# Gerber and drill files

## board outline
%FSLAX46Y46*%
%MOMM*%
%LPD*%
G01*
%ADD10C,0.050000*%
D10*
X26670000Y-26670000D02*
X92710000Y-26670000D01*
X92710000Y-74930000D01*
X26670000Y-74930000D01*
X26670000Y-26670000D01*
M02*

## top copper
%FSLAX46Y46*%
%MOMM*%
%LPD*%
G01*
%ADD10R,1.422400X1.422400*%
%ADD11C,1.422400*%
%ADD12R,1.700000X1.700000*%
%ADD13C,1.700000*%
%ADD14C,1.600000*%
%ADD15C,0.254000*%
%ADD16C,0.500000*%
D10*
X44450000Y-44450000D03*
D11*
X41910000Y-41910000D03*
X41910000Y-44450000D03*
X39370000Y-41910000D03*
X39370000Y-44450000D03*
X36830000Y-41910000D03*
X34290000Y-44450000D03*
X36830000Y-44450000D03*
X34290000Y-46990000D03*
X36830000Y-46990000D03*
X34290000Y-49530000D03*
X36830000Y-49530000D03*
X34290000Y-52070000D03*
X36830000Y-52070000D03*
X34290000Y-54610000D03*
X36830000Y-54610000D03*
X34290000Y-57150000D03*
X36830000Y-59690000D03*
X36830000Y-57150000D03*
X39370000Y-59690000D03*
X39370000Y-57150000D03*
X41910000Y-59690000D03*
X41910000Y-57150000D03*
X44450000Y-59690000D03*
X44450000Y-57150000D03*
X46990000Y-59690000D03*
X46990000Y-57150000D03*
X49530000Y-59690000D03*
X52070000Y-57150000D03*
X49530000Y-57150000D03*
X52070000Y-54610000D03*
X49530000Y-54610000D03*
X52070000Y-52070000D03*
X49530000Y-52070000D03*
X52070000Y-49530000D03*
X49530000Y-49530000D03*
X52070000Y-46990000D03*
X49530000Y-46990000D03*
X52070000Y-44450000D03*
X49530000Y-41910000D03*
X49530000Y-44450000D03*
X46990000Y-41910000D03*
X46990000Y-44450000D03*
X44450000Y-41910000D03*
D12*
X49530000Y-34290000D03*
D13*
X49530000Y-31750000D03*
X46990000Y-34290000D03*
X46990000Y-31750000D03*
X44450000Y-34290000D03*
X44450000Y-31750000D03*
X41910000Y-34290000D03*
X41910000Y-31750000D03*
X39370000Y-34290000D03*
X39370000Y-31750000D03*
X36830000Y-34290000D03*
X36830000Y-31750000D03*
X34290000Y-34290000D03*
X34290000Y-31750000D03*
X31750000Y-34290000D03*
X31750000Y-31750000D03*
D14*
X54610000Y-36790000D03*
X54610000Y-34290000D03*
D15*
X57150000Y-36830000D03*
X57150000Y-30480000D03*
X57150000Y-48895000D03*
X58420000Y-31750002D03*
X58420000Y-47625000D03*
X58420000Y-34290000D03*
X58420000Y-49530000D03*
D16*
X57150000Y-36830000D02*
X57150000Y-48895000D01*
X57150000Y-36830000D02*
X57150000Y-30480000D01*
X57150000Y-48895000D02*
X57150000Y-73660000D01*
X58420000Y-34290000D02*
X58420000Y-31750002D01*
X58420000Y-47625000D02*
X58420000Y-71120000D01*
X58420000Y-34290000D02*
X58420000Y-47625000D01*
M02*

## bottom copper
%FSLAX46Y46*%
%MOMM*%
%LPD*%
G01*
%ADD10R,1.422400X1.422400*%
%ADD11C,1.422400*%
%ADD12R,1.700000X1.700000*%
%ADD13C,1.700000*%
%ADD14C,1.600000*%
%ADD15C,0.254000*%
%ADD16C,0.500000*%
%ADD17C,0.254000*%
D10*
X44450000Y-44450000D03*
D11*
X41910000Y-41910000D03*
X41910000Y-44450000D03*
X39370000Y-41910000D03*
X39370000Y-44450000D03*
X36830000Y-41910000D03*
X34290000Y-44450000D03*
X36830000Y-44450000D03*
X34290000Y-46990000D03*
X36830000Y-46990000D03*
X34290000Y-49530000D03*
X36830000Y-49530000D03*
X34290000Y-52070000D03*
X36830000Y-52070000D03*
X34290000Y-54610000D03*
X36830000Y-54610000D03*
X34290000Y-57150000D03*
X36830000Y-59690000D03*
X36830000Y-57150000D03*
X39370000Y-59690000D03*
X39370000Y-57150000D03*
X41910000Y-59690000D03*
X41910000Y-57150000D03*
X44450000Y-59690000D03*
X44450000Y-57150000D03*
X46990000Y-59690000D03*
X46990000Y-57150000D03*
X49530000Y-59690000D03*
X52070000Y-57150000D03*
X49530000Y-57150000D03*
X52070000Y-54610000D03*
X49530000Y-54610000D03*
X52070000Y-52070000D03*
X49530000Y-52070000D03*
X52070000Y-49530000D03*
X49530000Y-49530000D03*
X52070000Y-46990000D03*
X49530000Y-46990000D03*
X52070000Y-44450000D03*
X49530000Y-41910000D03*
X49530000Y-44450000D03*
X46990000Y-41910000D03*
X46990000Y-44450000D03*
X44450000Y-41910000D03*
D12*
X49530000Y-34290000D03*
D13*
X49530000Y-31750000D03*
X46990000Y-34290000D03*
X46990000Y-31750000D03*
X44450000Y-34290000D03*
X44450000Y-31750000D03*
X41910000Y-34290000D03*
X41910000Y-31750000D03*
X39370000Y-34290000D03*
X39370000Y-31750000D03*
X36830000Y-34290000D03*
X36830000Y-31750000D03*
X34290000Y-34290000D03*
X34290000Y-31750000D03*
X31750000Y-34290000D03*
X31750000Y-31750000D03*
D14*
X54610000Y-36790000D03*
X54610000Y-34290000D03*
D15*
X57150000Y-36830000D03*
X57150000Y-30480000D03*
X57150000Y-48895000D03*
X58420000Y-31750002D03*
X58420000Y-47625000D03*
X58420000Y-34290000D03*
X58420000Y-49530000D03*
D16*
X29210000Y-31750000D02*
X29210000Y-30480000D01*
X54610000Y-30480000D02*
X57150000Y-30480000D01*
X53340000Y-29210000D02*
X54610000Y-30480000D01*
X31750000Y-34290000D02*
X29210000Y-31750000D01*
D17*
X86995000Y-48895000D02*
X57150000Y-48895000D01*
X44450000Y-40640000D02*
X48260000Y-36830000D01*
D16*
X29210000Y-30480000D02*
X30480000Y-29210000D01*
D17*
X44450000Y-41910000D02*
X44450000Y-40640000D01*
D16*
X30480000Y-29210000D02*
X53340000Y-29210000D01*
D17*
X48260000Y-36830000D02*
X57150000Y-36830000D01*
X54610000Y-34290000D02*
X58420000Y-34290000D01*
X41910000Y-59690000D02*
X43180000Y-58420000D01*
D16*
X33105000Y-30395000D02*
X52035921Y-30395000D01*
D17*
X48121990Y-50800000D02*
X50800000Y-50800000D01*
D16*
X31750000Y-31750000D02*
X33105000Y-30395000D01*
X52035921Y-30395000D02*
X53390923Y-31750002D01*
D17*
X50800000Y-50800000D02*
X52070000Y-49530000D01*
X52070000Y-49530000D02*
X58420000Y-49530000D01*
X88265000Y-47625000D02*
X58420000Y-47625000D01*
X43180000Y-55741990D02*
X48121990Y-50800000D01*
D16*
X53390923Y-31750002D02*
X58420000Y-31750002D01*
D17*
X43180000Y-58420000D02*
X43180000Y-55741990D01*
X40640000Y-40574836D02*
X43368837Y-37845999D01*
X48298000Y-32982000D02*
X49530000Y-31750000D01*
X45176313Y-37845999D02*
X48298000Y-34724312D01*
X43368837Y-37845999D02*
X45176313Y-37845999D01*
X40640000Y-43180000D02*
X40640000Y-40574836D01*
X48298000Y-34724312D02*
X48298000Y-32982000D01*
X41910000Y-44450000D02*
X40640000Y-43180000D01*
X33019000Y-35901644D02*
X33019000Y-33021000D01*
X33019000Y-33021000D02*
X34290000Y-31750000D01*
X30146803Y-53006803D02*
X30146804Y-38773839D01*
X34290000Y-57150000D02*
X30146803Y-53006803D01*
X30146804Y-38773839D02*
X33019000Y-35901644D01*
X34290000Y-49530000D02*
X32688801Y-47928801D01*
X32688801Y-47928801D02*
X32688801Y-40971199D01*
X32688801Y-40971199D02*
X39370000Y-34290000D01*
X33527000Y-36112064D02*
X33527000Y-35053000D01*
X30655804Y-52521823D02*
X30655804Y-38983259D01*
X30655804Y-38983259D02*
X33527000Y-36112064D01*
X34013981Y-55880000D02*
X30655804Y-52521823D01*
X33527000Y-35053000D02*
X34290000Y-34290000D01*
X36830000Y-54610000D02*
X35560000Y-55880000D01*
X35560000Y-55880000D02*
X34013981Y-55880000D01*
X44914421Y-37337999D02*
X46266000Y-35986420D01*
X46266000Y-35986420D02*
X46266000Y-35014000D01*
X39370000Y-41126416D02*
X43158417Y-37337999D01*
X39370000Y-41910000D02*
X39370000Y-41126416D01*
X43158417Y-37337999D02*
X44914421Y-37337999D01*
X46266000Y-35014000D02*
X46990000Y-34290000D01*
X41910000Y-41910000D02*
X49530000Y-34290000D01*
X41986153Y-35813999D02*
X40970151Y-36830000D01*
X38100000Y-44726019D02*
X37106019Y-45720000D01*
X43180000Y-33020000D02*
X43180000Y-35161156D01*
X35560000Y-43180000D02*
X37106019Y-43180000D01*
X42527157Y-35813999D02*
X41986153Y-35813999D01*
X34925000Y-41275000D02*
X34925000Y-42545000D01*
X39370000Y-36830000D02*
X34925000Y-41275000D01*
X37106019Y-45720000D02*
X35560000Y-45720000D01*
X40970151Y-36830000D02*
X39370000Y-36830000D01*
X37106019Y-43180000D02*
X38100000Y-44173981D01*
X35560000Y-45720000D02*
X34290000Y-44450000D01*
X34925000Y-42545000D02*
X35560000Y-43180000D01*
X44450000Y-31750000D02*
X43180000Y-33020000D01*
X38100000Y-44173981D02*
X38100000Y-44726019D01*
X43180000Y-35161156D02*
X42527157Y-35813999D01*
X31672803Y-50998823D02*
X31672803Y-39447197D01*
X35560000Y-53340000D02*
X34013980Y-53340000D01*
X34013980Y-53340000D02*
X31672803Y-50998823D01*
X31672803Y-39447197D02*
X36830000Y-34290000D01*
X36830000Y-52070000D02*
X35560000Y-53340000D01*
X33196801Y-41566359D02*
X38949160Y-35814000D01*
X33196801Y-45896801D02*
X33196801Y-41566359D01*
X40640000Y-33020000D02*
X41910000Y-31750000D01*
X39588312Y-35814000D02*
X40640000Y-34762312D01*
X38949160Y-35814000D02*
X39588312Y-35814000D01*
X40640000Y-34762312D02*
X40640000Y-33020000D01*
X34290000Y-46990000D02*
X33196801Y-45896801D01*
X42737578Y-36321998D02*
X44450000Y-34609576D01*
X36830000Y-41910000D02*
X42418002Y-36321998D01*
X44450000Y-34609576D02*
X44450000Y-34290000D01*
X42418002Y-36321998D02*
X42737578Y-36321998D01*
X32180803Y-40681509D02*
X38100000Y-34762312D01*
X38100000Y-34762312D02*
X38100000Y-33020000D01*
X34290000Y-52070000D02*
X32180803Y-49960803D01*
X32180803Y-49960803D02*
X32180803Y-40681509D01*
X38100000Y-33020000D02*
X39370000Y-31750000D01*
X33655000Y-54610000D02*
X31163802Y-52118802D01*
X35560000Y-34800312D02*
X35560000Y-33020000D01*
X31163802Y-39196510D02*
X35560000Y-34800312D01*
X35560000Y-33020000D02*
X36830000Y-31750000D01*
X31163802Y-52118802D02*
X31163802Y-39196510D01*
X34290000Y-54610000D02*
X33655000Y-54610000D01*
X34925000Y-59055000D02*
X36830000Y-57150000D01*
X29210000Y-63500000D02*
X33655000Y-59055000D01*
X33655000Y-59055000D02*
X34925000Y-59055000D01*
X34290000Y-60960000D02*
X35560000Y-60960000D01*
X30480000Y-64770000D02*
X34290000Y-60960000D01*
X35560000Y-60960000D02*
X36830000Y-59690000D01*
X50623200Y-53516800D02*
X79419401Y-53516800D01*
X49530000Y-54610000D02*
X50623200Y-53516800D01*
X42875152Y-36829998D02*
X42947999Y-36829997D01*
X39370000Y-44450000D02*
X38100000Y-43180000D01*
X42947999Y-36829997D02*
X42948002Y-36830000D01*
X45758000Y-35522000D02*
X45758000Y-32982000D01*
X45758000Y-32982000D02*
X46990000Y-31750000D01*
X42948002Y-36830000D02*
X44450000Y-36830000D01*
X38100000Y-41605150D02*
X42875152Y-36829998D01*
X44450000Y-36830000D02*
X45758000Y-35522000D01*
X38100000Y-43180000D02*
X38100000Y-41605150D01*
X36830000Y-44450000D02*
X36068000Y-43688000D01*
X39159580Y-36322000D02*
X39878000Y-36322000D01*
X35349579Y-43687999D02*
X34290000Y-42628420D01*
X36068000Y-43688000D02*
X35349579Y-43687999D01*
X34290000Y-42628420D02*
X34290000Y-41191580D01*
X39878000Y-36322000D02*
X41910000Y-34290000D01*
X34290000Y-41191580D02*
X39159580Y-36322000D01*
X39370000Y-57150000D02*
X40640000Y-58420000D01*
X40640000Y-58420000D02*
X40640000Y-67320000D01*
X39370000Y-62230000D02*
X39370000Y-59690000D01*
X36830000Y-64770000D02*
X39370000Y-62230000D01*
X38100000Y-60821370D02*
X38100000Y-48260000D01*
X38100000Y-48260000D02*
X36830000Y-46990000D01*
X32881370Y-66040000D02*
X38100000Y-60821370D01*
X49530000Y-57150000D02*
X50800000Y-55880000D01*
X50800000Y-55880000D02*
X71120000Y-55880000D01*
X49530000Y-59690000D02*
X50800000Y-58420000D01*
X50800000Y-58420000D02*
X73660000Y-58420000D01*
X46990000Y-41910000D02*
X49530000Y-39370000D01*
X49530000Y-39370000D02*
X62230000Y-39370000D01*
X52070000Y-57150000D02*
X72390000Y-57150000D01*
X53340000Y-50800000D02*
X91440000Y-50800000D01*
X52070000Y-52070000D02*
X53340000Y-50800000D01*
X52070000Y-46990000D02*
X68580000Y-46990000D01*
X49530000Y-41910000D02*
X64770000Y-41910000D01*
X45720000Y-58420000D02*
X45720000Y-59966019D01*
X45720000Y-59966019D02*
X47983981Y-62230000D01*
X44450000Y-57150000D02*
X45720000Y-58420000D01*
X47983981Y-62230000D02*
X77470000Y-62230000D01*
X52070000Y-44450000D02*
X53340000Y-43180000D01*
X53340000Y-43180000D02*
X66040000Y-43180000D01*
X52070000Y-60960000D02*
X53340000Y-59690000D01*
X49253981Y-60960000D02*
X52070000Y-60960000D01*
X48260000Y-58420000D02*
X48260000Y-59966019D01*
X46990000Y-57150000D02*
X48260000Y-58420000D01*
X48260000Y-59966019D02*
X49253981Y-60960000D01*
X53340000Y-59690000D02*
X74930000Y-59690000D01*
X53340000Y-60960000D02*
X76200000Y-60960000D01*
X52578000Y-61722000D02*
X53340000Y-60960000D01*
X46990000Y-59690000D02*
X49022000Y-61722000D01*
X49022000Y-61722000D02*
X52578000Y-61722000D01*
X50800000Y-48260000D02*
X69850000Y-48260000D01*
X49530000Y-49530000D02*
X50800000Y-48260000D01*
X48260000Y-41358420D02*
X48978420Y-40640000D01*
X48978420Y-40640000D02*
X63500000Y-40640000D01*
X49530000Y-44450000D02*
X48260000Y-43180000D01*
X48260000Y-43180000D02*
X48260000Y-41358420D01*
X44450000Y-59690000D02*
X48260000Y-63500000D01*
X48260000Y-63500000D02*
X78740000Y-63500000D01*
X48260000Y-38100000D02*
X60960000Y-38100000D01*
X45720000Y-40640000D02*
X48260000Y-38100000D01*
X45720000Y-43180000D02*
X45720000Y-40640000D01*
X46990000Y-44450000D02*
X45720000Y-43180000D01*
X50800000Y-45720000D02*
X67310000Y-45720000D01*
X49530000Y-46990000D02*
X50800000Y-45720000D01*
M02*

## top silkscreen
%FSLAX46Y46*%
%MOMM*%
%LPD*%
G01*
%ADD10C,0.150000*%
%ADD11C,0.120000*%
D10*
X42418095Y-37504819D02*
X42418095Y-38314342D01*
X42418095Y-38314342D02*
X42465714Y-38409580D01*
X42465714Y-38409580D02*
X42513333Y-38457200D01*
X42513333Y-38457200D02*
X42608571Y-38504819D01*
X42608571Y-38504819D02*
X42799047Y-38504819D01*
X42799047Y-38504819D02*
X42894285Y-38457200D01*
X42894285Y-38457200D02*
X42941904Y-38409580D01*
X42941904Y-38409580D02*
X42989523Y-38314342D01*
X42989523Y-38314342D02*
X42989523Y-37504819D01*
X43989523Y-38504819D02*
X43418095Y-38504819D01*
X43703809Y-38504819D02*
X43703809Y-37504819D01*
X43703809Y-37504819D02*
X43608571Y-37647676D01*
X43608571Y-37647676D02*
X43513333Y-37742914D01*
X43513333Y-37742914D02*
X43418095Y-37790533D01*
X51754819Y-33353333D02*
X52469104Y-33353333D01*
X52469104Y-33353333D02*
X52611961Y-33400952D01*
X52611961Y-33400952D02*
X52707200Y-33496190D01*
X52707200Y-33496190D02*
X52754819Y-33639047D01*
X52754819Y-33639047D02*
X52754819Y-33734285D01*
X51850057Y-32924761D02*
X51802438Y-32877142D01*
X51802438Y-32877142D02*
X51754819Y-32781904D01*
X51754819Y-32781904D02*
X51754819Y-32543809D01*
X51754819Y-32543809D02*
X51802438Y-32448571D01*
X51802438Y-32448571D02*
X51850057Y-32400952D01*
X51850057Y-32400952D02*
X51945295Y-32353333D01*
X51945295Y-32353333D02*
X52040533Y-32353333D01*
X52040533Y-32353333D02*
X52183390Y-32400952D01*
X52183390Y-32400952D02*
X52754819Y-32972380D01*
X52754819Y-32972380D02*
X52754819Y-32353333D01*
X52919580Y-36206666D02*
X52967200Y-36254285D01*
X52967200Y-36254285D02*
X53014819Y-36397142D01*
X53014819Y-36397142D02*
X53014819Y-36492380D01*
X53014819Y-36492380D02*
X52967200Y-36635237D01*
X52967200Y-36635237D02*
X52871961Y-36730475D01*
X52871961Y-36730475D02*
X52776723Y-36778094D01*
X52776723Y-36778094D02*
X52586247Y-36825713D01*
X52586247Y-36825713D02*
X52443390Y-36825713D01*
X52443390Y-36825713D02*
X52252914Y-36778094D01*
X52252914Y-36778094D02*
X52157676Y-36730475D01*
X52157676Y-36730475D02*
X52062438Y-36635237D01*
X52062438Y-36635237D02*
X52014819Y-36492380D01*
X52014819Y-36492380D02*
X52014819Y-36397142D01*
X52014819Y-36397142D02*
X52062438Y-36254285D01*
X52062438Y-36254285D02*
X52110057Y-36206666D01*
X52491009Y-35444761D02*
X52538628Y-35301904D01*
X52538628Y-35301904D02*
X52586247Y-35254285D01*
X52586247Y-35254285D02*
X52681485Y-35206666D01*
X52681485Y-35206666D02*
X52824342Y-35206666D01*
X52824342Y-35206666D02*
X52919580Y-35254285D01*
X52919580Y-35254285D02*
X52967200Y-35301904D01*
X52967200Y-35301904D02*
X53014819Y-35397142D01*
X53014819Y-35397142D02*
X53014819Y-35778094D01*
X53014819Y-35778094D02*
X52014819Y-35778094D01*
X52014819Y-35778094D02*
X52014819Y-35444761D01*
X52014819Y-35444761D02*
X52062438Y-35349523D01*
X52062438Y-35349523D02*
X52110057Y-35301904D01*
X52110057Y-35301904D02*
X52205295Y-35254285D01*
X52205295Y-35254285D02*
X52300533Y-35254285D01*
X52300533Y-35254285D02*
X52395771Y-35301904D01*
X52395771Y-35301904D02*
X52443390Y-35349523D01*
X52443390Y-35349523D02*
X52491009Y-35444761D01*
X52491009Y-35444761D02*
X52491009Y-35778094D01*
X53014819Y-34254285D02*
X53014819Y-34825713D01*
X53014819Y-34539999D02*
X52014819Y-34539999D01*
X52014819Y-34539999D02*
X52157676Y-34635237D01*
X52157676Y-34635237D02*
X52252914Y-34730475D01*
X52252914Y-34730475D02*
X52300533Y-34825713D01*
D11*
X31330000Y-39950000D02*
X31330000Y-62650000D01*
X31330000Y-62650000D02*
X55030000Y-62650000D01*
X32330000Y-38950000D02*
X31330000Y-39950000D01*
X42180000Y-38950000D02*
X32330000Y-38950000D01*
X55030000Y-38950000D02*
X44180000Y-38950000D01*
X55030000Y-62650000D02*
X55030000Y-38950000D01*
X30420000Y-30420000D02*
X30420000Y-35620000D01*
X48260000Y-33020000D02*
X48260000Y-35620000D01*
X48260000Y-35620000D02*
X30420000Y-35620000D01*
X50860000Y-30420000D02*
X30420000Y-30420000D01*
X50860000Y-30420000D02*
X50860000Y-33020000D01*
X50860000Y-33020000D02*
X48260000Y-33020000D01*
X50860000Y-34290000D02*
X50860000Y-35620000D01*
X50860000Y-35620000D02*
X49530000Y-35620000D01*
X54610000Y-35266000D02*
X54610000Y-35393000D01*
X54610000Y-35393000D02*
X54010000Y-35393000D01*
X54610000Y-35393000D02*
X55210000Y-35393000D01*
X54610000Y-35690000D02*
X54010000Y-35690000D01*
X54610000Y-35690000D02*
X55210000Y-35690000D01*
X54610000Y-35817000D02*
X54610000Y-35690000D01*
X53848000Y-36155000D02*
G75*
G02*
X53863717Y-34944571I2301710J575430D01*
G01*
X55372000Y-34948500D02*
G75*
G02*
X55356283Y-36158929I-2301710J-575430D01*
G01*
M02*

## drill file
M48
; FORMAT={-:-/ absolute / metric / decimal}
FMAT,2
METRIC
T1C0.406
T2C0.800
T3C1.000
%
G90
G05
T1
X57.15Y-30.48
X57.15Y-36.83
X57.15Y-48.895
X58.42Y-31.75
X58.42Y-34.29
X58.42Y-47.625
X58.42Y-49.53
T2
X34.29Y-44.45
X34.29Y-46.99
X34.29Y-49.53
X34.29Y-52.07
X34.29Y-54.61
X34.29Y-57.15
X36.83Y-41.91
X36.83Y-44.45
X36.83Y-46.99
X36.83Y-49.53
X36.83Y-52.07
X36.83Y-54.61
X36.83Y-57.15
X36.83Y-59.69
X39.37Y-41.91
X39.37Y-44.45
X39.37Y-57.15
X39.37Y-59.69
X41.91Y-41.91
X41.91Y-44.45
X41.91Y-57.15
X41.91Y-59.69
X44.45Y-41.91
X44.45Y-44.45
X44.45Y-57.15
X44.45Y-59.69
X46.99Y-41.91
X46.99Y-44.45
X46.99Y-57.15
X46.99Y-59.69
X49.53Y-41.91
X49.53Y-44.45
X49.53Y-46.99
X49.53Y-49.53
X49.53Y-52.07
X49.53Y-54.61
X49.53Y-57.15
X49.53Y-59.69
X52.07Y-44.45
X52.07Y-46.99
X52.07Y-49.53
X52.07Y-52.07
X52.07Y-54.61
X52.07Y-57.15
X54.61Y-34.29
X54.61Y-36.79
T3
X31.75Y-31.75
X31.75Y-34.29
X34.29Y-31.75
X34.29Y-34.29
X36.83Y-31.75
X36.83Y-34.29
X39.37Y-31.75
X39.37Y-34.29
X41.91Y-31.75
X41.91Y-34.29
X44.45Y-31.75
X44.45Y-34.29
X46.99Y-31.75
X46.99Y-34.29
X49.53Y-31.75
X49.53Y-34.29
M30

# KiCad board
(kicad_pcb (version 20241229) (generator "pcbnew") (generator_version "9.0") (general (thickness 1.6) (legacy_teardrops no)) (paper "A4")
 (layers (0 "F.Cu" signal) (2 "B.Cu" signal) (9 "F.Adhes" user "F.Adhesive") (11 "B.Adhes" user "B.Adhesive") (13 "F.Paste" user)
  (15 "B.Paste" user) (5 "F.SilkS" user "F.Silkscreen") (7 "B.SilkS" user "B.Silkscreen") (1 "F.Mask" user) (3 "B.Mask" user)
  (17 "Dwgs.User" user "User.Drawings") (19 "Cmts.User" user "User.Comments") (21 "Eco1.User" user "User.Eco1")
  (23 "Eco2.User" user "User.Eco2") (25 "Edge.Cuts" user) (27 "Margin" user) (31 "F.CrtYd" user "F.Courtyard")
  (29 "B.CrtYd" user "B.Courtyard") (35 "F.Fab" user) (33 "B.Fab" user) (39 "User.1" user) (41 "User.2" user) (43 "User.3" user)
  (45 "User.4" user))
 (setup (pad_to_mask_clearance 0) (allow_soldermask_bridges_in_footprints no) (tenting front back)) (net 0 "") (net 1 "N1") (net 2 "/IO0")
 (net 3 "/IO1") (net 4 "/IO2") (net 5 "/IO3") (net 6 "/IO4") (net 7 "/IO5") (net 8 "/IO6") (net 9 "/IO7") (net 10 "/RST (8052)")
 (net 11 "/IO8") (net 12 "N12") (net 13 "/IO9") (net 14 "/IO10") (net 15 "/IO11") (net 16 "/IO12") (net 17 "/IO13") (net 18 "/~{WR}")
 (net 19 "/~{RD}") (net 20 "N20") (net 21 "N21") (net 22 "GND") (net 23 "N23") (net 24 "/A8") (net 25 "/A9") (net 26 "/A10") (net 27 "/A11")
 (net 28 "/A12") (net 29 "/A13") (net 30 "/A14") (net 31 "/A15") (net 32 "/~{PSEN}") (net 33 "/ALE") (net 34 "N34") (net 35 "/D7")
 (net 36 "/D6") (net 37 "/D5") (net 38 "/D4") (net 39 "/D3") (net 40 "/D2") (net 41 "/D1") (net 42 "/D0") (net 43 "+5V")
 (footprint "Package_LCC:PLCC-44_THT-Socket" (layer "F.Cu") (at 44.45 44.45)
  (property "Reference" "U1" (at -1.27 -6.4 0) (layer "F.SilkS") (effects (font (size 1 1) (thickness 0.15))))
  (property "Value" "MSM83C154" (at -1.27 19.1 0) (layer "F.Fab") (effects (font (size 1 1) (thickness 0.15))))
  (fp_line (start -13.12 -4.5) (end -13.12 18.2) (stroke (width 0.12) (type solid)) (layer "F.SilkS"))
  (fp_line (start -13.12 18.2) (end 10.58 18.2) (stroke (width 0.12) (type solid)) (layer "F.SilkS"))
  (fp_line (start -12.12 -5.5) (end -13.12 -4.5) (stroke (width 0.12) (type solid)) (layer "F.SilkS"))
  (fp_line (start -2.27 -5.5) (end -12.12 -5.5) (stroke (width 0.12) (type solid)) (layer "F.SilkS"))
  (fp_line (start 10.58 -5.5) (end -0.27 -5.5) (stroke (width 0.12) (type solid)) (layer "F.SilkS"))
  (fp_line (start 10.58 18.2) (end 10.58 -5.5) (stroke (width 0.12) (type solid)) (layer "F.SilkS"))
  (pad "1" thru_hole rect (at 0 0) (size 1.4224 1.4224) (drill 0.8) (layers "*.Cu" "*.Mask") (remove_unused_layers no) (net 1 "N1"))
  (pad "2" thru_hole circle (at -2.54 -2.54) (size 1.4224 1.4224) (drill 0.8) (layers "*.Cu" "*.Mask") (remove_unused_layers no)
   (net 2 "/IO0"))
  (pad "3" thru_hole circle (at -2.54 0) (size 1.4224 1.4224) (drill 0.8) (layers "*.Cu" "*.Mask") (remove_unused_layers no) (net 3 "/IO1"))
  (pad "4" thru_hole circle (at -5.08 -2.54) (size 1.4224 1.4224) (drill 0.8) (layers "*.Cu" "*.Mask") (remove_unused_layers no)
   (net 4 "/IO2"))
  (pad "5" thru_hole circle (at -5.08 0) (size 1.4224 1.4224) (drill 0.8) (layers "*.Cu" "*.Mask") (remove_unused_layers no) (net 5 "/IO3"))
  (pad "6" thru_hole circle (at -7.62 -2.54) (size 1.4224 1.4224) (drill 0.8) (layers "*.Cu" "*.Mask") (remove_unused_layers no)
   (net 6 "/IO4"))
  (pad "7" thru_hole circle (at -10.16 0) (size 1.4224 1.4224) (drill 0.8) (layers "*.Cu" "*.Mask") (remove_unused_layers no) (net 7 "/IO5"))
  (pad "8" thru_hole circle (at -7.62 0) (size 1.4224 1.4224) (drill 0.8) (layers "*.Cu" "*.Mask") (remove_unused_layers no) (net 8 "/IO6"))
  (pad "9" thru_hole circle (at -10.16 2.54) (size 1.4224 1.4224) (drill 0.8) (layers "*.Cu" "*.Mask") (remove_unused_layers no)
   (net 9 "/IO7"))
  (pad "10" thru_hole circle (at -7.62 2.54) (size 1.4224 1.4224) (drill 0.8) (layers "*.Cu" "*.Mask") (remove_unused_layers no)
   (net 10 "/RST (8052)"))
  (pad "11" thru_hole circle (at -10.16 5.08) (size 1.4224 1.4224) (drill 0.8) (layers "*.Cu" "*.Mask") (remove_unused_layers no)
   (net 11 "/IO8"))
  (pad "12" thru_hole circle (at -7.62 5.08) (size 1.4224 1.4224) (drill 0.8) (layers "*.Cu" "*.Mask") (remove_unused_layers no)
   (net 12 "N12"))
  (pad "13" thru_hole circle (at -10.16 7.62) (size 1.4224 1.4224) (drill 0.8) (layers "*.Cu" "*.Mask") (remove_unused_layers no)
   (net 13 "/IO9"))
  (pad "14" thru_hole circle (at -7.62 7.62) (size 1.4224 1.4224) (drill 0.8) (layers "*.Cu" "*.Mask") (remove_unused_layers no)
   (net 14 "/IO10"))
  (pad "15" thru_hole circle (at -10.16 10.16) (size 1.4224 1.4224) (drill 0.8) (layers "*.Cu" "*.Mask") (remove_unused_layers no)
   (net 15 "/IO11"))
  (pad "16" thru_hole circle (at -7.62 10.16) (size 1.4224 1.4224) (drill 0.8) (layers "*.Cu" "*.Mask") (remove_unused_layers no)
   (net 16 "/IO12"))
  (pad "17" thru_hole circle (at -10.16 12.7) (size 1.4224 1.4224) (drill 0.8) (layers "*.Cu" "*.Mask") (remove_unused_layers no)
   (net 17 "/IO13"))
  (pad "18" thru_hole circle (at -7.62 15.24) (size 1.4224 1.4224) (drill 0.8) (layers "*.Cu" "*.Mask") (remove_unused_layers no)
   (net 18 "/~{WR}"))
  (pad "19" thru_hole circle (at -7.62 12.7) (size 1.4224 1.4224) (drill 0.8) (layers "*.Cu" "*.Mask") (remove_unused_layers no)
   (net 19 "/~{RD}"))
  (pad "20" thru_hole circle (at -5.08 15.24) (size 1.4224 1.4224) (drill 0.8) (layers "*.Cu" "*.Mask") (remove_unused_layers no)
   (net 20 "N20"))
  (pad "21" thru_hole circle (at -5.08 12.7) (size 1.4224 1.4224) (drill 0.8) (layers "*.Cu" "*.Mask") (remove_unused_layers no)
   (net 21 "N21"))
  (pad "22" thru_hole circle (at -2.54 15.24) (size 1.4224 1.4224) (drill 0.8) (layers "*.Cu" "*.Mask") (remove_unused_layers no)
   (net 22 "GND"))
  (pad "23" thru_hole circle (at -2.54 12.7) (size 1.4224 1.4224) (drill 0.8) (layers "*.Cu" "*.Mask") (remove_unused_layers no)
   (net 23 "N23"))
  (pad "24" thru_hole circle (at 0 15.24) (size 1.4224 1.4224) (drill 0.8) (layers "*.Cu" "*.Mask") (remove_unused_layers no) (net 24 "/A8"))
  (pad "25" thru_hole circle (at 0 12.7) (size 1.4224 1.4224) (drill 0.8) (layers "*.Cu" "*.Mask") (remove_unused_layers no) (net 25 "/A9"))
  (pad "26" thru_hole circle (at 2.54 15.24) (size 1.4224 1.4224) (drill 0.8) (layers "*.Cu" "*.Mask") (remove_unused_layers no)
   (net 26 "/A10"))
  (pad "27" thru_hole circle (at 2.54 12.7) (size 1.4224 1.4224) (drill 0.8) (layers "*.Cu" "*.Mask") (remove_unused_layers no)
   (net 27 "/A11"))
  (pad "28" thru_hole circle (at 5.08 15.24) (size 1.4224 1.4224) (drill 0.8) (layers "*.Cu" "*.Mask") (remove_unused_layers no)
   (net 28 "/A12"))
  (pad "29" thru_hole circle (at 7.62 12.7) (size 1.4224 1.4224) (drill 0.8) (layers "*.Cu" "*.Mask") (remove_unused_layers no)
   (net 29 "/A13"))
  (pad "30" thru_hole circle (at 5.08 12.7) (size 1.4224 1.4224) (drill 0.8) (layers "*.Cu" "*.Mask") (remove_unused_layers no)
   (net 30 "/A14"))
  (pad "31" thru_hole circle (at 7.62 10.16) (size 1.4224 1.4224) (drill 0.8) (layers "*.Cu" "*.Mask") (remove_unused_layers no)
   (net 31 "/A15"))
  (pad "32" thru_hole circle (at 5.08 10.16) (size 1.4224 1.4224) (drill 0.8) (layers "*.Cu" "*.Mask") (remove_unused_layers no)
   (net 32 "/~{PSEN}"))
  (pad "33" thru_hole circle (at 7.62 7.62) (size 1.4224 1.4224) (drill 0.8) (layers "*.Cu" "*.Mask") (remove_unused_layers no)
   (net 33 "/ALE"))
  (pad "34" thru_hole circle (at 5.08 7.62) (size 1.4224 1.4224) (drill 0.8) (layers "*.Cu" "*.Mask") (remove_unused_layers no)
   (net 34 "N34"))
  (pad "35" thru_hole circle (at 7.62 5.08) (size 1.4224 1.4224) (drill 0.8) (layers "*.Cu" "*.Mask") (remove_unused_layers no)
   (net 22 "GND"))
  (pad "36" thru_hole circle (at 5.08 5.08) (size 1.4224 1.4224) (drill 0.8) (layers "*.Cu" "*.Mask") (remove_unused_layers no)
   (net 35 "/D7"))
  (pad "37" thru_hole circle (at 7.62 2.54) (size 1.4224 1.4224) (drill 0.8) (layers "*.Cu" "*.Mask") (remove_unused_layers no)
   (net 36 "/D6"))
  (pad "38" thru_hole circle (at 5.08 2.54) (size 1.4224 1.4224) (drill 0.8) (layers "*.Cu" "*.Mask") (remove_unused_layers no)
   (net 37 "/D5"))
  (pad "39" thru_hole circle (at 7.62 0) (size 1.4224 1.4224) (drill 0.8) (layers "*.Cu" "*.Mask") (remove_unused_layers no) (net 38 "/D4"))
  (pad "40" thru_hole circle (at 5.08 -2.54) (size 1.4224 1.4224) (drill 0.8) (layers "*.Cu" "*.Mask") (remove_unused_layers no)
   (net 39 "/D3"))
  (pad "41" thru_hole circle (at 5.08 0) (size 1.4224 1.4224) (drill 0.8) (layers "*.Cu" "*.Mask") (remove_unused_layers no) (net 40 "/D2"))
  (pad "42" thru_hole circle (at 2.54 -2.54) (size 1.4224 1.4224) (drill 0.8) (layers "*.Cu" "*.Mask") (remove_unused_layers no)
   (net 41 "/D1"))
  (pad "43" thru_hole circle (at 2.54 0) (size 1.4224 1.4224) (drill 0.8) (layers "*.Cu" "*.Mask") (remove_unused_layers no) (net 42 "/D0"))
  (pad "44" thru_hole circle (at 0 -2.54) (size 1.4224 1.4224) (drill 0.8) (layers "*.Cu" "*.Mask") (remove_unused_layers no) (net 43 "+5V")))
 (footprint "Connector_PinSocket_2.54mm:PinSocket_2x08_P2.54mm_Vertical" (layer "F.Cu") (at 49.53 34.29 -90)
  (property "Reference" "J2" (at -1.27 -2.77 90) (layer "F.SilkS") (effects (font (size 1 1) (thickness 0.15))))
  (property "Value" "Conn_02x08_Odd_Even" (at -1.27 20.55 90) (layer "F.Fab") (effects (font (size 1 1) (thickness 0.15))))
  (fp_line (start -3.87 19.11) (end 1.33 19.11) (stroke (width 0.12) (type solid)) (layer "F.SilkS"))
  (fp_line (start -1.27 1.27) (end 1.33 1.27) (stroke (width 0.12) (type solid)) (layer "F.SilkS"))
  (fp_line (start 1.33 1.27) (end 1.33 19.11) (stroke (width 0.12) (type solid)) (layer "F.SilkS"))
  (fp_line (start -3.87 -1.33) (end -3.87 19.11) (stroke (width 0.12) (type solid)) (layer "F.SilkS"))
  (fp_line (start -3.87 -1.33) (end -1.27 -1.33) (stroke (width 0.12) (type solid)) (layer "F.SilkS"))
  (fp_line (start -1.27 -1.33) (end -1.27 1.27) (stroke (width 0.12) (type solid)) (layer "F.SilkS"))
  (fp_line (start 0 -1.33) (end 1.33 -1.33) (stroke (width 0.12) (type solid)) (layer "F.SilkS"))
  (fp_line (start 1.33 -1.33) (end 1.33 0) (stroke (width 0.12) (type solid)) (layer "F.SilkS"))
  (pad "1" thru_hole rect (at 0 0 270) (size 1.7 1.7) (drill 1) (layers "*.Cu" "*.Mask") (remove_unused_layers no) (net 2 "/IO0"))
  (pad "2" thru_hole circle (at -2.54 0 270) (size 1.7 1.7) (drill 1) (layers "*.Cu" "*.Mask") (remove_unused_layers no) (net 3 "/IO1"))
  (pad "3" thru_hole circle (at 0 2.54 270) (size 1.7 1.7) (drill 1) (layers "*.Cu" "*.Mask") (remove_unused_layers no) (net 4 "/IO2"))
  (pad "4" thru_hole circle (at -2.54 2.54 270) (size 1.7 1.7) (drill 1) (layers "*.Cu" "*.Mask") (remove_unused_layers no) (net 5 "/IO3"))
  (pad "5" thru_hole circle (at 0 5.08 270) (size 1.7 1.7) (drill 1) (layers "*.Cu" "*.Mask") (remove_unused_layers no) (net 6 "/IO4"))
  (pad "6" thru_hole circle (at -2.54 5.08 270) (size 1.7 1.7) (drill 1) (layers "*.Cu" "*.Mask") (remove_unused_layers no) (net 7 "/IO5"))
  (pad "7" thru_hole circle (at 0 7.62 270) (size 1.7 1.7) (drill 1) (layers "*.Cu" "*.Mask") (remove_unused_layers no) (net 8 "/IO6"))
  (pad "8" thru_hole circle (at -2.54 7.62 270) (size 1.7 1.7) (drill 1) (layers "*.Cu" "*.Mask") (remove_unused_layers no) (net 9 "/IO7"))
  (pad "9" thru_hole circle (at 0 10.16 270) (size 1.7 1.7) (drill 1) (layers "*.Cu" "*.Mask") (remove_unused_layers no) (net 11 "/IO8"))
  (pad "10" thru_hole circle (at -2.54 10.16 270) (size 1.7 1.7) (drill 1) (layers "*.Cu" "*.Mask") (remove_unused_layers no)
   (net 13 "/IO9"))
  (pad "11" thru_hole circle (at 0 12.7 270) (size 1.7 1.7) (drill 1) (layers "*.Cu" "*.Mask") (remove_unused_layers no) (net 14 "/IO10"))
  (pad "12" thru_hole circle (at -2.54 12.7 270) (size 1.7 1.7) (drill 1) (layers "*.Cu" "*.Mask") (remove_unused_layers no)
   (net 15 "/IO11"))
  (pad "13" thru_hole circle (at 0 15.24 270) (size 1.7 1.7) (drill 1) (layers "*.Cu" "*.Mask") (remove_unused_layers no) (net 16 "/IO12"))
  (pad "14" thru_hole circle (at -2.54 15.24 270) (size 1.7 1.7) (drill 1) (layers "*.Cu" "*.Mask") (remove_unused_layers no)
   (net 17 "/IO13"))
  (pad "15" thru_hole circle (at 0 17.78 270) (size 1.7 1.7) (drill 1) (layers "*.Cu" "*.Mask") (remove_unused_layers no) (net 43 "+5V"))
  (pad "16" thru_hole circle (at -2.54 17.78 270) (size 1.7 1.7) (drill 1) (layers "*.Cu" "*.Mask") (remove_unused_layers no) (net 22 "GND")))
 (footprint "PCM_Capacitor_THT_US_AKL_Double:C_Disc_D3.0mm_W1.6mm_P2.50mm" (layer "F.Cu") (at 54.61 36.79 90)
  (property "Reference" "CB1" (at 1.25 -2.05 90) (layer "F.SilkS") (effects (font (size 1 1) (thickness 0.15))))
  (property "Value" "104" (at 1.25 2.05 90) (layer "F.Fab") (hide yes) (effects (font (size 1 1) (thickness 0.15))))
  (fp_line (start 1.524 0) (end 1.397 0) (stroke (width 0.12) (type solid)) (layer "F.SilkS"))
  (fp_line (start 1.397 0) (end 1.397 -0.6) (stroke (width 0.12) (type solid)) (layer "F.SilkS"))
  (fp_line (start 1.397 0) (end 1.397 0.6) (stroke (width 0.12) (type solid)) (layer "F.SilkS"))
  (fp_line (start 1.1 0) (end 1.1 -0.6) (stroke (width 0.12) (type solid)) (layer "F.SilkS"))
  (fp_line (start 1.1 0) (end 1.1 0.6) (stroke (width 0.12) (type solid)) (layer "F.SilkS"))
  (fp_line (start 0.973 0) (end 1.1 0) (stroke (width 0.12) (type solid)) (layer "F.SilkS"))
  (fp_arc (start 0.635 -0.762) (mid 1.241234 -0.832639) (end 1.845429 -0.746283) (stroke (width 0.12) (type solid)) (layer "F.SilkS"))
  (fp_arc (start 1.8415 0.762) (mid 1.235266 0.832639) (end 0.631071 0.746283) (stroke (width 0.12) (type solid)) (layer "F.SilkS"))
  (pad "1" thru_hole circle (at 0 0 90) (size 1.6 1.6) (drill 0.8) (layers "*.Cu" "*.Mask") (remove_unused_layers no) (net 43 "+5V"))
  (pad "2" thru_hole circle (at 2.5 0 90) (size 1.6 1.6) (drill 0.8) (layers "*.Cu" "*.Mask") (remove_unused_layers no) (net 22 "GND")))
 (gr_rect (start 26.67 26.67) (end 92.71 74.93) (stroke (width 0.05) (type default)) (fill no) (layer "Edge.Cuts"))
 (segment (start 57.15 36.83) (end 57.15 48.895) (width 0.5) (layer "F.Cu") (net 43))
 (segment (start 57.15 36.83) (end 57.15 30.48) (width 0.5) (layer "F.Cu") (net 43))
 (segment (start 57.15 48.895) (end 57.15 73.66) (width 0.5) (layer "F.Cu") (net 43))
 (via (at 57.15 36.83) (size 0.254) (drill 0.4064) (layers "F.Cu" "B.Cu") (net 43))
 (via (at 57.15 30.48) (size 0.254) (drill 0.4064) (layers "F.Cu" "B.Cu") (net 43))
 (via (at 57.15 48.895) (size 0.254) (drill 0.4064) (layers "F.Cu" "B.Cu") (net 43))
 (segment (start 29.21 31.75) (end 29.21 30.48) (width 0.5) (layer "B.Cu") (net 43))
 (segment (start 54.61 30.48) (end 57.15 30.48) (width 0.5) (layer "B.Cu") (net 43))
 (segment (start 53.34 29.21) (end 54.61 30.48) (width 0.5) (layer "B.Cu") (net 43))
 (segment (start 31.75 34.29) (end 29.21 31.75) (width 0.5) (layer "B.Cu") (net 43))
 (segment (start 86.995 48.895) (end 57.15 48.895) (width 0.254) (layer "B.Cu") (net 43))
 (segment (start 44.45 40.64) (end 48.26 36.83) (width 0.254) (layer "B.Cu") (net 43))
 (segment (start 29.21 30.48) (end 30.48 29.21) (width 0.5) (layer "B.Cu") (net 43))
 (segment (start 44.45 41.91) (end 44.45 40.64) (width 0.254) (layer "B.Cu") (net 43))
 (segment (start 30.48 29.21) (end 53.34 29.21) (width 0.5) (layer "B.Cu") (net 43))
 (segment (start 48.26 36.83) (end 57.15 36.83) (width 0.254) (layer "B.Cu") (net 43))
 (segment (start 58.42 34.29) (end 58.42 31.750002) (width 0.5) (layer "F.Cu") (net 22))
 (segment (start 58.42 47.625) (end 58.42 71.12) (width 0.5) (layer "F.Cu") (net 22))
 (segment (start 58.42 34.29) (end 58.42 47.625) (width 0.5) (layer "F.Cu") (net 22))
 (via (at 58.42 31.750002) (size 0.254) (drill 0.4064) (layers "F.Cu" "B.Cu") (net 22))
 (via (at 58.42 47.625) (size 0.254) (drill 0.4064) (layers "F.Cu" "B.Cu") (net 22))
 (via (at 58.42 34.29) (size 0.254) (drill 0.4064) (layers "F.Cu" "B.Cu") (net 22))
 (via (at 58.42 49.53) (size 0.254) (drill 0.4064) (layers "F.Cu" "B.Cu") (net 22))
 (segment (start 54.61 34.29) (end 58.42 34.29) (width 0.254) (layer "B.Cu") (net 22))
 (segment (start 41.91 59.69) (end 43.18 58.42) (width 0.254) (layer "B.Cu") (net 22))
 (segment (start 33.105 30.395) (end 52.035921 30.395) (width 0.5) (layer "B.Cu") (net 22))
 (segment (start 48.12199 50.8) (end 50.8 50.8) (width 0.254) (layer "B.Cu") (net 22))
 (segment (start 31.75 31.75) (end 33.105 30.395) (width 0.5) (layer "B.Cu") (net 22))
 (segment (start 52.035921 30.395) (end 53.390923 31.750002) (width 0.5) (layer "B.Cu") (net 22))
 (segment (start 50.8 50.8) (end 52.07 49.53) (width 0.254) (layer "B.Cu") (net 22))
 (segment (start 52.07 49.53) (end 58.42 49.53) (width 0.254) (layer "B.Cu") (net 22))
 (segment (start 88.265 47.625) (end 58.42 47.625) (width 0.254) (layer "B.Cu") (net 22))
 (segment (start 43.18 55.74199) (end 48.12199 50.8) (width 0.254) (layer "B.Cu") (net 22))
 (segment (start 53.390923 31.750002) (end 58.42 31.750002) (width 0.5) (layer "B.Cu") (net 22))
 (segment (start 43.18 58.42) (end 43.18 55.74199) (width 0.254) (layer "B.Cu") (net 22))
 (segment (start 40.64 40.574836) (end 43.368837 37.845999) (width 0.254) (layer "B.Cu") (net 3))
 (segment (start 48.298 32.982) (end 49.53 31.75) (width 0.254) (layer "B.Cu") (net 3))
 (segment (start 45.176313 37.845999) (end 48.298 34.724312) (width 0.254) (layer "B.Cu") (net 3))
 (segment (start 43.368837 37.845999) (end 45.176313 37.845999) (width 0.254) (layer "B.Cu") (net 3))
 (segment (start 40.64 43.18) (end 40.64 40.574836) (width 0.254) (layer "B.Cu") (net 3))
 (segment (start 48.298 34.724312) (end 48.298 32.982) (width 0.254) (layer "B.Cu") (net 3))
 (segment (start 41.91 44.45) (end 40.64 43.18) (width 0.254) (layer "B.Cu") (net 3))
 (segment (start 33.019 35.901644) (end 33.019 33.021) (width 0.254) (layer "B.Cu") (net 17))
 (segment (start 33.019 33.021) (end 34.29 31.75) (width 0.254) (layer "B.Cu") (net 17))
 (segment (start 30.146803 53.006803) (end 30.146804 38.773839) (width 0.254) (layer "B.Cu") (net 17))
 (segment (start 34.29 57.15) (end 30.146803 53.006803) (width 0.254) (layer "B.Cu") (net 17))
 (segment (start 30.146804 38.773839) (end 33.019 35.901644) (width 0.254) (layer "B.Cu") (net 17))
 (segment (start 34.29 49.53) (end 32.688801 47.928801) (width 0.254) (layer "B.Cu") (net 11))
 (segment (start 32.688801 47.928801) (end 32.688801 40.971199) (width 0.254) (layer "B.Cu") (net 11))
 (segment (start 32.688801 40.971199) (end 39.37 34.29) (width 0.254) (layer "B.Cu") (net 11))
 (segment (start 33.527 36.112064) (end 33.527 35.053) (width 0.254) (layer "B.Cu") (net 16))
 (segment (start 30.655804 52.521823) (end 30.655804 38.983259) (width 0.254) (layer "B.Cu") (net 16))
 (segment (start 30.655804 38.983259) (end 33.527 36.112064) (width 0.254) (layer "B.Cu") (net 16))
 (segment (start 34.013981 55.88) (end 30.655804 52.521823) (width 0.254) (layer "B.Cu") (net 16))
 (segment (start 33.527 35.053) (end 34.29 34.29) (width 0.254) (layer "B.Cu") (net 16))
 (segment (start 36.83 54.61) (end 35.56 55.88) (width 0.254) (layer "B.Cu") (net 16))
 (segment (start 35.56 55.88) (end 34.013981 55.88) (width 0.254) (layer "B.Cu") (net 16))
 (segment (start 44.914421 37.337999) (end 46.266 35.98642) (width 0.254) (layer "B.Cu") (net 4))
 (segment (start 46.266 35.98642) (end 46.266 35.014) (width 0.254) (layer "B.Cu") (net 4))
 (segment (start 39.37 41.126416) (end 43.158417 37.337999) (width 0.254) (layer "B.Cu") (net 4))
 (segment (start 39.37 41.91) (end 39.37 41.126416) (width 0.254) (layer "B.Cu") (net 4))
 (segment (start 43.158417 37.337999) (end 44.914421 37.337999) (width 0.254) (layer "B.Cu") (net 4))
 (segment (start 46.266 35.014) (end 46.99 34.29) (width 0.254) (layer "B.Cu") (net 4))
 (segment (start 41.91 41.91) (end 49.53 34.29) (width 0.254) (layer "B.Cu") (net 2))
 (segment (start 41.986153 35.813999) (end 40.970151 36.83) (width 0.254) (layer "B.Cu") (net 7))
 (segment (start 38.1 44.726019) (end 37.106019 45.72) (width 0.254) (layer "B.Cu") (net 7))
 (segment (start 43.18 33.02) (end 43.18 35.161156) (width 0.254) (layer "B.Cu") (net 7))
 (segment (start 35.56 43.18) (end 37.106019 43.18) (width 0.254) (layer "B.Cu") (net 7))
 (segment (start 42.527157 35.813999) (end 41.986153 35.813999) (width 0.254) (layer "B.Cu") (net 7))
 (segment (start 34.925 41.275) (end 34.925 42.545) (width 0.254) (layer "B.Cu") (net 7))
 (segment (start 39.37 36.83) (end 34.925 41.275) (width 0.254) (layer "B.Cu") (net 7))
 (segment (start 37.106019 45.72) (end 35.56 45.72) (width 0.254) (layer "B.Cu") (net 7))
 (segment (start 40.970151 36.83) (end 39.37 36.83) (width 0.254) (layer "B.Cu") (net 7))
 (segment (start 37.106019 43.18) (end 38.1 44.173981) (width 0.254) (layer "B.Cu") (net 7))
 (segment (start 35.56 45.72) (end 34.29 44.45) (width 0.254) (layer "B.Cu") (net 7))
 (segment (start 34.925 42.545) (end 35.56 43.18) (width 0.254) (layer "B.Cu") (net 7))
 (segment (start 44.45 31.75) (end 43.18 33.02) (width 0.254) (layer "B.Cu") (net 7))
 (segment (start 38.1 44.173981) (end 38.1 44.726019) (width 0.254) (layer "B.Cu") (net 7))
 (segment (start 43.18 35.161156) (end 42.527157 35.813999) (width 0.254) (layer "B.Cu") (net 7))
 (segment (start 31.672803 50.998823) (end 31.672803 39.447197) (width 0.254) (layer "B.Cu") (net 14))
 (segment (start 35.56 53.34) (end 34.01398 53.34) (width 0.254) (layer "B.Cu") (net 14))
 (segment (start 34.01398 53.34) (end 31.672803 50.998823) (width 0.254) (layer "B.Cu") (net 14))
 (segment (start 31.672803 39.447197) (end 36.83 34.29) (width 0.254) (layer "B.Cu") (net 14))
 (segment (start 36.83 52.07) (end 35.56 53.34) (width 0.254) (layer "B.Cu") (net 14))
 (segment (start 33.196801 41.566359) (end 38.94916 35.814) (width 0.254) (layer "B.Cu") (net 9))
 (segment (start 33.196801 45.896801) (end 33.196801 41.566359) (width 0.254) (layer "B.Cu") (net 9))
 (segment (start 40.64 33.02) (end 41.91 31.75) (width 0.254) (layer "B.Cu") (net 9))
 (segment (start 39.588312 35.814) (end 40.64 34.762312) (width 0.254) (layer "B.Cu") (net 9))
 (segment (start 38.94916 35.814) (end 39.588312 35.814) (width 0.254) (layer "B.Cu") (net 9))
 (segment (start 40.64 34.762312) (end 40.64 33.02) (width 0.254) (layer "B.Cu") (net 9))
 (segment (start 34.29 46.99) (end 33.196801 45.896801) (width 0.254) (layer "B.Cu") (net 9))
 (segment (start 42.737578 36.321998) (end 44.45 34.609576) (width 0.254) (layer "B.Cu") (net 6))
 (segment (start 36.83 41.91) (end 42.418002 36.321998) (width 0.254) (layer "B.Cu") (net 6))
 (segment (start 44.45 34.609576) (end 44.45 34.29) (width 0.254) (layer "B.Cu") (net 6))
 (segment (start 42.418002 36.321998) (end 42.737578 36.321998) (width 0.254) (layer "B.Cu") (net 6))
 (segment (start 32.180803 40.681509) (end 38.1 34.762312) (width 0.254) (layer "B.Cu") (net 13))
 (segment (start 38.1 34.762312) (end 38.1 33.02) (width 0.254) (layer "B.Cu") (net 13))
 (segment (start 34.29 52.07) (end 32.180803 49.960803) (width 0.254) (layer "B.Cu") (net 13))
 (segment (start 32.180803 49.960803) (end 32.180803 40.681509) (width 0.254) (layer "B.Cu") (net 13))
 (segment (start 38.1 33.02) (end 39.37 31.75) (width 0.254) (layer "B.Cu") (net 13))
 (segment (start 33.655 54.61) (end 31.163802 52.118802) (width 0.254) (layer "B.Cu") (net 15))
 (segment (start 35.56 34.800312) (end 35.56 33.02) (width 0.254) (layer "B.Cu") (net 15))
 (segment (start 31.163802 39.19651) (end 35.56 34.800312) (width 0.254) (layer "B.Cu") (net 15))
 (segment (start 35.56 33.02) (end 36.83 31.75) (width 0.254) (layer "B.Cu") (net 15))
 (segment (start 31.163802 52.118802) (end 31.163802 39.19651) (width 0.254) (layer "B.Cu") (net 15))
 (segment (start 34.29 54.61) (end 33.655 54.61) (width 0.254) (layer "B.Cu") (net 15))
 (segment (start 34.925 59.055) (end 36.83 57.15) (width 0.254) (layer "B.Cu") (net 19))
 (segment (start 29.21 63.5) (end 33.655 59.055) (width 0.254) (layer "B.Cu") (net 19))
 (segment (start 33.655 59.055) (end 34.925 59.055) (width 0.254) (layer "B.Cu") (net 19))
 (segment (start 34.29 60.96) (end 35.56 60.96) (width 0.254) (layer "B.Cu") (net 18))
 (segment (start 30.48 64.77) (end 34.29 60.96) (width 0.254) (layer "B.Cu") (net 18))
 (segment (start 35.56 60.96) (end 36.83 59.69) (width 0.254) (layer "B.Cu") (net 18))
 (segment (start 50.6232 53.5168) (end 79.419401 53.5168) (width 0.254) (layer "B.Cu") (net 32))
 (segment (start 49.53 54.61) (end 50.6232 53.5168) (width 0.254) (layer "B.Cu") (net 32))
 (segment (start 42.875152 36.829998) (end 42.947999 36.829997) (width 0.254) (layer "B.Cu") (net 5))
 (segment (start 39.37 44.45) (end 38.1 43.18) (width 0.254) (layer "B.Cu") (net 5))
 (segment (start 42.947999 36.829997) (end 42.948002 36.83) (width 0.254) (layer "B.Cu") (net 5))
 (segment (start 45.758 35.522) (end 45.758 32.982) (width 0.254) (layer "B.Cu") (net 5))
 (segment (start 45.758 32.982) (end 46.99 31.75) (width 0.254) (layer "B.Cu") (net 5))
 (segment (start 42.948002 36.83) (end 44.45 36.83) (width 0.254) (layer "B.Cu") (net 5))
 (segment (start 38.1 41.60515) (end 42.875152 36.829998) (width 0.254) (layer "B.Cu") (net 5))
 (segment (start 44.45 36.83) (end 45.758 35.522) (width 0.254) (layer "B.Cu") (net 5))
 (segment (start 38.1 43.18) (end 38.1 41.60515) (width 0.254) (layer "B.Cu") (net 5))
 (segment (start 36.83 44.45) (end 36.068 43.688) (width 0.254) (layer "B.Cu") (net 8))
 (segment (start 39.15958 36.322) (end 39.878 36.322) (width 0.254) (layer "B.Cu") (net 8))
 (segment (start 35.349579 43.687999) (end 34.29 42.62842) (width 0.254) (layer "B.Cu") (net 8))
 (segment (start 36.068 43.688) (end 35.349579 43.687999) (width 0.254) (layer "B.Cu") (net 8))
 (segment (start 34.29 42.62842) (end 34.29 41.19158) (width 0.254) (layer "B.Cu") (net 8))
 (segment (start 39.878 36.322) (end 41.91 34.29) (width 0.254) (layer "B.Cu") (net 8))
 (segment (start 34.29 41.19158) (end 39.15958 36.322) (width 0.254) (layer "B.Cu") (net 8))
 (segment (start 39.37 57.15) (end 40.64 58.42) (width 0.254) (layer "B.Cu") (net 21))
 (segment (start 40.64 58.42) (end 40.64 67.32) (width 0.254) (layer "B.Cu") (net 21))
 (segment (start 39.37 62.23) (end 39.37 59.69) (width 0.254) (layer "B.Cu") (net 20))
 (segment (start 36.83 64.77) (end 39.37 62.23) (width 0.254) (layer "B.Cu") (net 20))
 (segment (start 38.1 60.82137) (end 38.1 48.26) (width 0.254) (layer "B.Cu") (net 10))
 (segment (start 38.1 48.26) (end 36.83 46.99) (width 0.254) (layer "B.Cu") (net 10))
 (segment (start 32.88137 66.04) (end 38.1 60.82137) (width 0.254) (layer "B.Cu") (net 10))
 (segment (start 49.53 57.15) (end 50.8 55.88) (width 0.254) (layer "B.Cu") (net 30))
 (segment (start 50.8 55.88) (end 71.12 55.88) (width 0.254) (layer "B.Cu") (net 30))
 (segment (start 49.53 59.69) (end 50.8 58.42) (width 0.254) (layer "B.Cu") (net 28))
 (segment (start 50.8 58.42) (end 73.66 58.42) (width 0.254) (layer "B.Cu") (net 28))
 (segment (start 46.99 41.91) (end 49.53 39.37) (width 0.254) (layer "B.Cu") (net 41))
 (segment (start 49.53 39.37) (end 62.23 39.37) (width 0.254) (layer "B.Cu") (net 41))
 (segment (start 52.07 57.15) (end 72.39 57.15) (width 0.254) (layer "B.Cu") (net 29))
 (segment (start 53.34 50.8) (end 91.44 50.8) (width 0.254) (layer "B.Cu") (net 33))
 (segment (start 52.07 52.07) (end 53.34 50.8) (width 0.254) (layer "B.Cu") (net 33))
 (segment (start 52.07 46.99) (end 68.58 46.99) (width 0.254) (layer "B.Cu") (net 36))
 (segment (start 49.53 41.91) (end 64.77 41.91) (width 0.254) (layer "B.Cu") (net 39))
 (segment (start 45.72 58.42) (end 45.72 59.966019) (width 0.254) (layer "B.Cu") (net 25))
 (segment (start 45.72 59.966019) (end 47.983981 62.23) (width 0.254) (layer "B.Cu") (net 25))
 (segment (start 44.45 57.15) (end 45.72 58.42) (width 0.254) (layer "B.Cu") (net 25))
 (segment (start 47.983981 62.23) (end 77.47 62.23) (width 0.254) (layer "B.Cu") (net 25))
 (segment (start 52.07 44.45) (end 53.34 43.18) (width 0.254) (layer "B.Cu") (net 38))
 (segment (start 53.34 43.18) (end 66.04 43.18) (width 0.254) (layer "B.Cu") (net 38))
 (segment (start 52.07 60.96) (end 53.34 59.69) (width 0.254) (layer "B.Cu") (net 27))
 (segment (start 49.253981 60.96) (end 52.07 60.96) (width 0.254) (layer "B.Cu") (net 27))
 (segment (start 48.26 58.42) (end 48.26 59.966019) (width 0.254) (layer "B.Cu") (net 27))
 (segment (start 46.99 57.15) (end 48.26 58.42) (width 0.254) (layer "B.Cu") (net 27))
 (segment (start 48.26 59.966019) (end 49.253981 60.96) (width 0.254) (layer "B.Cu") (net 27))
 (segment (start 53.34 59.69) (end 74.93 59.69) (width 0.254) (layer "B.Cu") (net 27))
 (segment (start 53.34 60.96) (end 76.2 60.96) (width 0.254) (layer "B.Cu") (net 26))
 (segment (start 52.578 61.722) (end 53.34 60.96) (width 0.254) (layer "B.Cu") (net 26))
 (segment (start 46.99 59.69) (end 49.022 61.722) (width 0.254) (layer "B.Cu") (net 26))
 (segment (start 49.022 61.722) (end 52.578 61.722) (width 0.254) (layer "B.Cu") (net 26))
 (segment (start 50.8 48.26) (end 69.85 48.26) (width 0.254) (layer "B.Cu") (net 35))
 (segment (start 49.53 49.53) (end 50.8 48.26) (width 0.254) (layer "B.Cu") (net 35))
 (segment (start 48.26 41.35842) (end 48.97842 40.64) (width 0.254) (layer "B.Cu") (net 40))
 (segment (start 48.97842 40.64) (end 63.5 40.64) (width 0.254) (layer "B.Cu") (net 40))
 (segment (start 49.53 44.45) (end 48.26 43.18) (width 0.254) (layer "B.Cu") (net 40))
 (segment (start 48.26 43.18) (end 48.26 41.35842) (width 0.254) (layer "B.Cu") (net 40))
 (segment (start 44.45 59.69) (end 48.26 63.5) (width 0.254) (layer "B.Cu") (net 24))
 (segment (start 48.26 63.5) (end 78.74 63.5) (width 0.254) (layer "B.Cu") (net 24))
 (segment (start 48.26 38.1) (end 60.96 38.1) (width 0.254) (layer "B.Cu") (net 42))
 (segment (start 45.72 40.64) (end 48.26 38.1) (width 0.254) (layer "B.Cu") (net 42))
 (segment (start 45.72 43.18) (end 45.72 40.64) (width 0.254) (layer "B.Cu") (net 42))
 (segment (start 46.99 44.45) (end 45.72 43.18) (width 0.254) (layer "B.Cu") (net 42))
 (segment (start 50.8 45.72) (end 67.31 45.72) (width 0.254) (layer "B.Cu") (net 37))
 (segment (start 49.53 46.99) (end 50.8 45.72) (width 0.254) (layer "B.Cu") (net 37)))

